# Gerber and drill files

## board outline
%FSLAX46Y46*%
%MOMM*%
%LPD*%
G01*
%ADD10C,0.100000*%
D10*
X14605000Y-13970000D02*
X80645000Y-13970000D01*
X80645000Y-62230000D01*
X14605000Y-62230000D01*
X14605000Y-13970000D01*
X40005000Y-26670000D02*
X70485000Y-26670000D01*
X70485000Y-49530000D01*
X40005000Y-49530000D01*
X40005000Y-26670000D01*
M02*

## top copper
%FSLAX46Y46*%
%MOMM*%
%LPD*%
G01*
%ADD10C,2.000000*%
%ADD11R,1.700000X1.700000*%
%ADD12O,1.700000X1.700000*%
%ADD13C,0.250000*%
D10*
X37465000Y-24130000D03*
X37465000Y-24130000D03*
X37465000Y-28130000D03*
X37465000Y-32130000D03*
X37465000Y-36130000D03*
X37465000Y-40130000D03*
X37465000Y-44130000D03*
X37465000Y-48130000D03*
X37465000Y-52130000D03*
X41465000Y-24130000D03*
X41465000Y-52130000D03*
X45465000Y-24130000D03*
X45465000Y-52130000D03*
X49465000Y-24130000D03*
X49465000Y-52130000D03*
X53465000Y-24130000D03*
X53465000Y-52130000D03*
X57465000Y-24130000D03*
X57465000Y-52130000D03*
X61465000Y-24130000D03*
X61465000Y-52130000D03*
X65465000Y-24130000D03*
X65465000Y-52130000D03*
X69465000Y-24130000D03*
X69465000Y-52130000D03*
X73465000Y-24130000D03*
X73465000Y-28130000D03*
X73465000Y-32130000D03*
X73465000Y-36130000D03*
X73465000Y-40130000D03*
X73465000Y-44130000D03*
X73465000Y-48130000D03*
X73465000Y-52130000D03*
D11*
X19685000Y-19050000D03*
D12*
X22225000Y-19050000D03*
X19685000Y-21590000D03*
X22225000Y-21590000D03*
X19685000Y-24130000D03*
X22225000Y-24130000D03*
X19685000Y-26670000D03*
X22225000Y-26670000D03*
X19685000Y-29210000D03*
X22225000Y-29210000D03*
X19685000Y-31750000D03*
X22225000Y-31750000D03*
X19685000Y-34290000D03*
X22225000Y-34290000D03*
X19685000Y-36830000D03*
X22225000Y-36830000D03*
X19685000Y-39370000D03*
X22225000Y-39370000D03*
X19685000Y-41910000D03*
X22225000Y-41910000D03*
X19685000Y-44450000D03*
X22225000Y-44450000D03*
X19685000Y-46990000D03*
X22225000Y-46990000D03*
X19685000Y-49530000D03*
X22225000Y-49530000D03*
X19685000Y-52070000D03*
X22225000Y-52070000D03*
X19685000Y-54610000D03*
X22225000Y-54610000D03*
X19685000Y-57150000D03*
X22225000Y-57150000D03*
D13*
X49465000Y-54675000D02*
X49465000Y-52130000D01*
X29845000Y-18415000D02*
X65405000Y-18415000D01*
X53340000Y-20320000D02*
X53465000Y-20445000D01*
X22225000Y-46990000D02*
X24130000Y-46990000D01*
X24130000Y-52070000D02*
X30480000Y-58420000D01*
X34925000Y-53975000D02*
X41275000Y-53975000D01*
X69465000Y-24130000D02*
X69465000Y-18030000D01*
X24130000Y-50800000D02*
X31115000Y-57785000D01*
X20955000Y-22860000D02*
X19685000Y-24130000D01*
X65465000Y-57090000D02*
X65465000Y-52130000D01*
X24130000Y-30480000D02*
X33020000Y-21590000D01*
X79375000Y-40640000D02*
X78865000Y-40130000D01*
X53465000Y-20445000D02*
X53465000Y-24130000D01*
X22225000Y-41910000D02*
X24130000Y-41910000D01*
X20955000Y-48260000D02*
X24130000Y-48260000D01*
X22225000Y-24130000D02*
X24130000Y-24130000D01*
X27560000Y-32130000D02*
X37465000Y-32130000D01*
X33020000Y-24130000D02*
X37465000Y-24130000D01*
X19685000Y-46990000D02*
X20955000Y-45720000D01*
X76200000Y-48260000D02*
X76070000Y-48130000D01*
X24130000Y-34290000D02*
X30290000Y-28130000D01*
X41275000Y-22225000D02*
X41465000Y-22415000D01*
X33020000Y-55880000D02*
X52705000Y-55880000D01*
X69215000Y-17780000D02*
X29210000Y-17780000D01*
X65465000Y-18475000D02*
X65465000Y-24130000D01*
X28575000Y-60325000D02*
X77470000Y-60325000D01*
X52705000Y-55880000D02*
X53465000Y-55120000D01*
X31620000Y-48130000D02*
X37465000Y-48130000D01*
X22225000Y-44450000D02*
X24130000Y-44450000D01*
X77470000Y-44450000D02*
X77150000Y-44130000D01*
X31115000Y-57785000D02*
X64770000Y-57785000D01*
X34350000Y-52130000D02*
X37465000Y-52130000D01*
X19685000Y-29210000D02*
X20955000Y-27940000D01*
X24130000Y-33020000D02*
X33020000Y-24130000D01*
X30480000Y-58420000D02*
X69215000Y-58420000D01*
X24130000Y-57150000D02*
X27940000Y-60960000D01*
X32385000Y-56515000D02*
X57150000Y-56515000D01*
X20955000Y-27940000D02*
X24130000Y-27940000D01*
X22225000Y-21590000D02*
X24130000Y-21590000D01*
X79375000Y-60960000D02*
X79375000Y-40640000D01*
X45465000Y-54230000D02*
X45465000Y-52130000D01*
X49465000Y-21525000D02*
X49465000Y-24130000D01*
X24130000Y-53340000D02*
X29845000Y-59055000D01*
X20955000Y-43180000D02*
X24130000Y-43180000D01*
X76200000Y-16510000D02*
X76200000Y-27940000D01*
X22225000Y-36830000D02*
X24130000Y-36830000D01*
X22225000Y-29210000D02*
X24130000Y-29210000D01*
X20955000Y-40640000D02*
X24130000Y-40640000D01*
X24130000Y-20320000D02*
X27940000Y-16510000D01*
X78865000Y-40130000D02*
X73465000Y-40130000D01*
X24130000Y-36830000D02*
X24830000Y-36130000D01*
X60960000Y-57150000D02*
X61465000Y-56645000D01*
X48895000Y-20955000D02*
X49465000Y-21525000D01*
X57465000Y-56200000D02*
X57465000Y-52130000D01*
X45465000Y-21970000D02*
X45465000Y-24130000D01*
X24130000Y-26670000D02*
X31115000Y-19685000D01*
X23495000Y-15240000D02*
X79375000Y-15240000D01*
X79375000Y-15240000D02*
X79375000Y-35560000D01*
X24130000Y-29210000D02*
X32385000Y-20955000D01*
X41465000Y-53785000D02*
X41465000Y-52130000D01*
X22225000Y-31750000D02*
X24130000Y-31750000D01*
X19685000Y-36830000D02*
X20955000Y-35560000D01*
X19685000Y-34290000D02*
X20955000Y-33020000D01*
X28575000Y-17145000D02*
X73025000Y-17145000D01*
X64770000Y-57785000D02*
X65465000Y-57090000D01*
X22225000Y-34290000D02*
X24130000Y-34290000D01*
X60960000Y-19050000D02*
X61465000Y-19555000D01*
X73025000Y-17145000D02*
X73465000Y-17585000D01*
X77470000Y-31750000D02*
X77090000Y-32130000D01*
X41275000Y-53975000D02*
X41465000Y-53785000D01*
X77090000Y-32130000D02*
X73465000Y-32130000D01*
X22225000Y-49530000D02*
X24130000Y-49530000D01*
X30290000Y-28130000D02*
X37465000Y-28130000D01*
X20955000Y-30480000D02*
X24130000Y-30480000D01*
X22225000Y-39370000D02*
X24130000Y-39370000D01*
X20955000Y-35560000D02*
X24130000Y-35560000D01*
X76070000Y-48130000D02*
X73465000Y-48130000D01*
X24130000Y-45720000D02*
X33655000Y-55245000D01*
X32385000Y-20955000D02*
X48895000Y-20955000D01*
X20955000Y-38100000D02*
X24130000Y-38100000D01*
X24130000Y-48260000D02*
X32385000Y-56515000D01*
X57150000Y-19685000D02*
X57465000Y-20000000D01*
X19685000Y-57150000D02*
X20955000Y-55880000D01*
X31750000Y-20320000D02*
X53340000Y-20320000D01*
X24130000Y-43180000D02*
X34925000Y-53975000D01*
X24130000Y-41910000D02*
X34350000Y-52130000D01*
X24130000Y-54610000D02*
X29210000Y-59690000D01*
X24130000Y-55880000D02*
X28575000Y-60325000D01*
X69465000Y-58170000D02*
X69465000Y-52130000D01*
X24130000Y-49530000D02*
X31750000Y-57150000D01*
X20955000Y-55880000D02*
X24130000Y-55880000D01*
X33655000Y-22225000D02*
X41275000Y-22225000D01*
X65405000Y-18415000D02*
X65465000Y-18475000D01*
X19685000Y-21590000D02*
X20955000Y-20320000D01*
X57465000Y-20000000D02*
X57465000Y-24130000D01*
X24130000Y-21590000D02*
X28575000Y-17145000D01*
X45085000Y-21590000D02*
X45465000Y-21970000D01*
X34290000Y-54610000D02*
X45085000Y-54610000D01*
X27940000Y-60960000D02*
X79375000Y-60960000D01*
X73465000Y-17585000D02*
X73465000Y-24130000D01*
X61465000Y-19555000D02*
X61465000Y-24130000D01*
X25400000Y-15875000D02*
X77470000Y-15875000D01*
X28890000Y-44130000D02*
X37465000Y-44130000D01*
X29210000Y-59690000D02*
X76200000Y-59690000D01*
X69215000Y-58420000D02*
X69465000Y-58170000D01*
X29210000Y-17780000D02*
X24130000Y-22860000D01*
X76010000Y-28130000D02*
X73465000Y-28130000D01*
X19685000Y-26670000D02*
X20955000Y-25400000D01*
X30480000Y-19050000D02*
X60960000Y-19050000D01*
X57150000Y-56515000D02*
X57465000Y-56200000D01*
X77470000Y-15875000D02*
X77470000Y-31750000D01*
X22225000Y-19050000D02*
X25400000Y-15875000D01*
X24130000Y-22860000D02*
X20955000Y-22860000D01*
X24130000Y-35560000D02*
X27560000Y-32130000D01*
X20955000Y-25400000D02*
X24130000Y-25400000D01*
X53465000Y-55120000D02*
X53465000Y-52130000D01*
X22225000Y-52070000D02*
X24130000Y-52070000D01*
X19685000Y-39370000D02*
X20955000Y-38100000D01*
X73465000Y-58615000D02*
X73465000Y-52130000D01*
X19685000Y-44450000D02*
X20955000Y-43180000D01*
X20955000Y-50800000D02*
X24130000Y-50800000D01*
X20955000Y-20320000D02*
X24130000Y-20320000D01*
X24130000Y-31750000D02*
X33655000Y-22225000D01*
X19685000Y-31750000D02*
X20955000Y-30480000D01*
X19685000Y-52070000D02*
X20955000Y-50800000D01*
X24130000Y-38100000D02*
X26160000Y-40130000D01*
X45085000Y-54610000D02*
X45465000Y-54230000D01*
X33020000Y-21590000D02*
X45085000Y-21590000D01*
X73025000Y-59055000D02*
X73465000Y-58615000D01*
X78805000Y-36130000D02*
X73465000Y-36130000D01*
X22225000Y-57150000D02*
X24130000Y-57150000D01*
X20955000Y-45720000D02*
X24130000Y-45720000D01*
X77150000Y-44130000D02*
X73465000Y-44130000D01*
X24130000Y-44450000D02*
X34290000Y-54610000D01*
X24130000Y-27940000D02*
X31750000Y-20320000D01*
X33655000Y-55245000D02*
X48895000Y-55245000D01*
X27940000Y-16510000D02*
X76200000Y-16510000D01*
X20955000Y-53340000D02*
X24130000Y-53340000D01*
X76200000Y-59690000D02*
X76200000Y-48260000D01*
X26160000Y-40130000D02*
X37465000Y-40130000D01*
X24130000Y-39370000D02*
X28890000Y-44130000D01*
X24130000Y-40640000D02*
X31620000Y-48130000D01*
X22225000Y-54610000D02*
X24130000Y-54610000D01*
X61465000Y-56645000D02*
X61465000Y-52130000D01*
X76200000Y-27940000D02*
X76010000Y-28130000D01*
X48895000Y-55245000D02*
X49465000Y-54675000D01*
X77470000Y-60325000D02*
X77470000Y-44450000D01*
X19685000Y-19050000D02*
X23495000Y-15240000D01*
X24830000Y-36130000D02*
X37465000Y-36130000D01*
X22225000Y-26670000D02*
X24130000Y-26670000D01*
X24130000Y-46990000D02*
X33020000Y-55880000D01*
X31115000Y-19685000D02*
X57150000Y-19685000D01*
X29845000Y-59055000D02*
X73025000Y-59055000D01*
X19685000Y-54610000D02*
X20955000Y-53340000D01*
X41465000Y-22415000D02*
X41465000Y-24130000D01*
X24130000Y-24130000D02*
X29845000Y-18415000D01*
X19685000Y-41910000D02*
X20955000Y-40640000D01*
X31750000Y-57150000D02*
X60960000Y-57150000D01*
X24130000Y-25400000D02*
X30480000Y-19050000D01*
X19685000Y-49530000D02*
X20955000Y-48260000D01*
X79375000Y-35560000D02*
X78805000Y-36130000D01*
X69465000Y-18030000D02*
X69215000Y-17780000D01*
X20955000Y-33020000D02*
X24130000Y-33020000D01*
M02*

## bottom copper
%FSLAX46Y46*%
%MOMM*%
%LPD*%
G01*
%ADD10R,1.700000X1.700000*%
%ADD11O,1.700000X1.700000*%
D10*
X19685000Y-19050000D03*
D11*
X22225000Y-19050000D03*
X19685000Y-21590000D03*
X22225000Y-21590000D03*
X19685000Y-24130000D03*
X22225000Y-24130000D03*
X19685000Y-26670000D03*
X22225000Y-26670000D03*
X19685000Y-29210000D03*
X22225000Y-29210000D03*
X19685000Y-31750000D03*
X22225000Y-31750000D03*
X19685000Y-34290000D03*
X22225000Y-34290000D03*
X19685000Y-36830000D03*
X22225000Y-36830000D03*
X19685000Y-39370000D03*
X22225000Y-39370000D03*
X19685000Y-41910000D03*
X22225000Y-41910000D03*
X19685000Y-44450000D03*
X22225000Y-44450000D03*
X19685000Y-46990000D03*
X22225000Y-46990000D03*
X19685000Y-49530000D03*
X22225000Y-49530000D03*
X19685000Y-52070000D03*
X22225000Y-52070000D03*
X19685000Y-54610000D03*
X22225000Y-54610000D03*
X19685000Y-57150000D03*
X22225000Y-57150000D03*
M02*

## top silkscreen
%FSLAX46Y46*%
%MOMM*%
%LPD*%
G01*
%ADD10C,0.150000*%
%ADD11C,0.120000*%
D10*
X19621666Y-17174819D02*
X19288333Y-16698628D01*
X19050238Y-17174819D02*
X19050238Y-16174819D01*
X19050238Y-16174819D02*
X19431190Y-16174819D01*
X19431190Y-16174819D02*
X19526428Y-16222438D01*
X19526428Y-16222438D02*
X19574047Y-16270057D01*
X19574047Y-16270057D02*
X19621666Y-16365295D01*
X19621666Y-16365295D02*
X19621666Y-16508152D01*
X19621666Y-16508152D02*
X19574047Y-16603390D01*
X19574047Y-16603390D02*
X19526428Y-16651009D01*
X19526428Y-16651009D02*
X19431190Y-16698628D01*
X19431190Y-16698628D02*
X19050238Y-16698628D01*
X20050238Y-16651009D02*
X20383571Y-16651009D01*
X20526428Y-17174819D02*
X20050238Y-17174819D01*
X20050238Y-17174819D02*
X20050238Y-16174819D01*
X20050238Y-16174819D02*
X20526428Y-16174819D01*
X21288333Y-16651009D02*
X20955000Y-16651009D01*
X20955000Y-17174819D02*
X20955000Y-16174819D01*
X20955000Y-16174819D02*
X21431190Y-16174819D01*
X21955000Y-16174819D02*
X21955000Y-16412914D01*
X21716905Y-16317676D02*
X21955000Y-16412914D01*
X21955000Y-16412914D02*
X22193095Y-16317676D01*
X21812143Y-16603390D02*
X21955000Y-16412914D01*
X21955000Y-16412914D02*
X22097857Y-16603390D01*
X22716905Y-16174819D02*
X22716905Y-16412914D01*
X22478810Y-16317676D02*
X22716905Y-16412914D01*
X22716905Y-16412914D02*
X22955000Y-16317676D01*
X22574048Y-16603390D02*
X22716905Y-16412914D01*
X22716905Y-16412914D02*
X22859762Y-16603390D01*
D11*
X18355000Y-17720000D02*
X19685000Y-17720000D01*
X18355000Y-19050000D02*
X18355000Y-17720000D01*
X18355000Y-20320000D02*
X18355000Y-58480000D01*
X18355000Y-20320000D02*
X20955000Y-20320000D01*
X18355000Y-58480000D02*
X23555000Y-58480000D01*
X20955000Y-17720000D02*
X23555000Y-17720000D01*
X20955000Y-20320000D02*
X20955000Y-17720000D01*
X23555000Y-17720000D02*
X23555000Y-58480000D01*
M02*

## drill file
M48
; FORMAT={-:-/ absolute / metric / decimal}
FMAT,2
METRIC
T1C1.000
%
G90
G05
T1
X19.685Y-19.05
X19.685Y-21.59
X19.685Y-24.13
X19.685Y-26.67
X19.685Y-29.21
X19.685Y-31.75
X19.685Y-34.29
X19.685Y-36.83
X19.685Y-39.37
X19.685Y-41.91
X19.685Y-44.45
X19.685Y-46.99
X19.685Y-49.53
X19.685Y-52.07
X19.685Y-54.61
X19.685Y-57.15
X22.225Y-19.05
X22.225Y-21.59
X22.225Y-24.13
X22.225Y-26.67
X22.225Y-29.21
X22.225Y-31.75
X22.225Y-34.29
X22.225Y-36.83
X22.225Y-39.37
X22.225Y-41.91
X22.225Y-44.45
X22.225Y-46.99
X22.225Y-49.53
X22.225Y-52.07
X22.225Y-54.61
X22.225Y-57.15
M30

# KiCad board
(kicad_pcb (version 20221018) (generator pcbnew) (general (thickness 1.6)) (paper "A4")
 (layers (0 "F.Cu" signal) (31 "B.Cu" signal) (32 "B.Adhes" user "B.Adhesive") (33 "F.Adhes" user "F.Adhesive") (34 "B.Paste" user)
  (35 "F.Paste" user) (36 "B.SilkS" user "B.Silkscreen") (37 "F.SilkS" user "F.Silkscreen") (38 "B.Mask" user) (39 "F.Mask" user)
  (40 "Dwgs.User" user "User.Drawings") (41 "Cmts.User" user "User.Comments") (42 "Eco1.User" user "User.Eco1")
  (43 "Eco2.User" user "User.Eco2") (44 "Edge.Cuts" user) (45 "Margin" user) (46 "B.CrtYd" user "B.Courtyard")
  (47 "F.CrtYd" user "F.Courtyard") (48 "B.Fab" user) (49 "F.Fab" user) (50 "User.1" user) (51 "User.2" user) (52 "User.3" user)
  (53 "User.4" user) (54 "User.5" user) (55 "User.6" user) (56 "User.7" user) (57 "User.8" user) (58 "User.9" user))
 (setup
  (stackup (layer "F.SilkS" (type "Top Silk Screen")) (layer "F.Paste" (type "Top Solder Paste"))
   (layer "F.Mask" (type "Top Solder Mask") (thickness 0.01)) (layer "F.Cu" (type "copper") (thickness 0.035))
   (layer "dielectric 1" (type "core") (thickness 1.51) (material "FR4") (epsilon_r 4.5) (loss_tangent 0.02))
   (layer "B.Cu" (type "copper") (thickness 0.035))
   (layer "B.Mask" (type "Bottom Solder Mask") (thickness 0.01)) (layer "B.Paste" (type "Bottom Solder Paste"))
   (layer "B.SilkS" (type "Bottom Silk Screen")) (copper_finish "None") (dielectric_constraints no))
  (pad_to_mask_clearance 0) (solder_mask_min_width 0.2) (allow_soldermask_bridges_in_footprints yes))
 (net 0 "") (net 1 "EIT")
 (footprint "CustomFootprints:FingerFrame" (layer "F.Cu") (at 37.465 24.13)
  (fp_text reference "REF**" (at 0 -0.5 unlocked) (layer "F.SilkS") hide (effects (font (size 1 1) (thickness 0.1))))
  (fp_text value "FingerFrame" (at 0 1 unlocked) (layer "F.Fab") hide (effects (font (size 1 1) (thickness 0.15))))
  (pad "1" smd circle (at 0 0) (size 2 2) (layers "F.Cu" "F.Paste" "F.Mask") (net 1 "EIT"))
  (pad "1" smd circle (at 0 0) (size 2 2) (layers "F.Cu" "F.Paste" "F.Mask") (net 1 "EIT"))
  (pad "1" smd circle (at 0 4) (size 2 2) (layers "F.Cu" "F.Paste" "F.Mask") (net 1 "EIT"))
  (pad "1" smd circle (at 0 8) (size 2 2) (layers "F.Cu" "F.Paste" "F.Mask") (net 1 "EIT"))
  (pad "1" smd circle (at 0 12) (size 2 2) (layers "F.Cu" "F.Paste" "F.Mask") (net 1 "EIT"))
  (pad "1" smd circle (at 0 16) (size 2 2) (layers "F.Cu" "F.Paste" "F.Mask") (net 1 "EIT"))
  (pad "1" smd circle (at 0 20) (size 2 2) (layers "F.Cu" "F.Paste" "F.Mask") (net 1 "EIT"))
  (pad "1" smd circle (at 0 24) (size 2 2) (layers "F.Cu" "F.Paste" "F.Mask") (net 1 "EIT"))
  (pad "1" smd circle (at 0 28) (size 2 2) (layers "F.Cu" "F.Paste" "F.Mask") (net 1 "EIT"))
  (pad "1" smd circle (at 4 0) (size 2 2) (layers "F.Cu" "F.Paste" "F.Mask") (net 1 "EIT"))
  (pad "1" smd circle (at 4 28) (size 2 2) (layers "F.Cu" "F.Paste" "F.Mask") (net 1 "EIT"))
  (pad "1" smd circle (at 8 0) (size 2 2) (layers "F.Cu" "F.Paste" "F.Mask") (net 1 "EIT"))
  (pad "1" smd circle (at 8 28) (size 2 2) (layers "F.Cu" "F.Paste" "F.Mask") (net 1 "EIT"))
  (pad "1" smd circle (at 12 0) (size 2 2) (layers "F.Cu" "F.Paste" "F.Mask") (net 1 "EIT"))
  (pad "1" smd circle (at 12 28) (size 2 2) (layers "F.Cu" "F.Paste" "F.Mask") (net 1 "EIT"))
  (pad "1" smd circle (at 16 0) (size 2 2) (layers "F.Cu" "F.Paste" "F.Mask") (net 1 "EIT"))
  (pad "1" smd circle (at 16 28) (size 2 2) (layers "F.Cu" "F.Paste" "F.Mask") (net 1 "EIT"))
  (pad "1" smd circle (at 20 0) (size 2 2) (layers "F.Cu" "F.Paste" "F.Mask") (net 1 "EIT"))
  (pad "1" smd circle (at 20 28) (size 2 2) (layers "F.Cu" "F.Paste" "F.Mask") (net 1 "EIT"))
  (pad "1" smd circle (at 24 0) (size 2 2) (layers "F.Cu" "F.Paste" "F.Mask") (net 1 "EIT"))
  (pad "1" smd circle (at 24 28) (size 2 2) (layers "F.Cu" "F.Paste" "F.Mask") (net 1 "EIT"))
  (pad "1" smd circle (at 28 0) (size 2 2) (layers "F.Cu" "F.Paste" "F.Mask") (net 1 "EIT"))
  (pad "1" smd circle (at 28 28) (size 2 2) (layers "F.Cu" "F.Paste" "F.Mask") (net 1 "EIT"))
  (pad "1" smd circle (at 32 0) (size 2 2) (layers "F.Cu" "F.Paste" "F.Mask") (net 1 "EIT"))
  (pad "1" smd circle (at 32 28) (size 2 2) (layers "F.Cu" "F.Paste" "F.Mask") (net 1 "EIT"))
  (pad "1" smd circle (at 36 0) (size 2 2) (layers "F.Cu" "F.Paste" "F.Mask") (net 1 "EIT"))
  (pad "1" smd circle (at 36 4) (size 2 2) (layers "F.Cu" "F.Paste" "F.Mask") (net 1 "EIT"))
  (pad "1" smd circle (at 36 8) (size 2 2) (layers "F.Cu" "F.Paste" "F.Mask") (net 1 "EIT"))
  (pad "1" smd circle (at 36 12) (size 2 2) (layers "F.Cu" "F.Paste" "F.Mask") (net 1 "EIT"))
  (pad "1" smd circle (at 36 16) (size 2 2) (layers "F.Cu" "F.Paste" "F.Mask") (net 1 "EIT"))
  (pad "1" smd circle (at 36 20) (size 2 2) (layers "F.Cu" "F.Paste" "F.Mask") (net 1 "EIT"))
  (pad "1" smd circle (at 36 24) (size 2 2) (layers "F.Cu" "F.Paste" "F.Mask") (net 1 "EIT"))
  (pad "1" smd circle (at 36 28) (size 2 2) (layers "F.Cu" "F.Paste" "F.Mask") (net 1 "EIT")))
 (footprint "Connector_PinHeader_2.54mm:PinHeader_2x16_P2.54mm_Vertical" (layer "F.Cu") (at 19.685 19.05)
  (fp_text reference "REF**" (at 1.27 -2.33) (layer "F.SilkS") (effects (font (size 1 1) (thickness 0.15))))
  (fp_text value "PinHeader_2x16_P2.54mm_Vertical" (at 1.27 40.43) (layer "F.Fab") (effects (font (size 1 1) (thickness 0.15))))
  (fp_line (start -1.33 -1.33) (end 0 -1.33) (stroke (width 0.12) (type solid)) (layer "F.SilkS"))
  (fp_line (start -1.33 0) (end -1.33 -1.33) (stroke (width 0.12) (type solid)) (layer "F.SilkS"))
  (fp_line (start -1.33 1.27) (end -1.33 39.43) (stroke (width 0.12) (type solid)) (layer "F.SilkS"))
  (fp_line (start -1.33 1.27) (end 1.27 1.27) (stroke (width 0.12) (type solid)) (layer "F.SilkS"))
  (fp_line (start -1.33 39.43) (end 3.87 39.43) (stroke (width 0.12) (type solid)) (layer "F.SilkS"))
  (fp_line (start 1.27 -1.33) (end 3.87 -1.33) (stroke (width 0.12) (type solid)) (layer "F.SilkS"))
  (fp_line (start 1.27 1.27) (end 1.27 -1.33) (stroke (width 0.12) (type solid)) (layer "F.SilkS"))
  (fp_line (start 3.87 -1.33) (end 3.87 39.43) (stroke (width 0.12) (type solid)) (layer "F.SilkS"))
  (pad "1" thru_hole rect (at 0 0) (size 1.7 1.7) (drill 1) (layers "*.Cu" "*.Mask") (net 1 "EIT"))
  (pad "2" thru_hole oval (at 2.54 0) (size 1.7 1.7) (drill 1) (layers "*.Cu" "*.Mask") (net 1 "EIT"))
  (pad "3" thru_hole oval (at 0 2.54) (size 1.7 1.7) (drill 1) (layers "*.Cu" "*.Mask") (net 1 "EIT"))
  (pad "4" thru_hole oval (at 2.54 2.54) (size 1.7 1.7) (drill 1) (layers "*.Cu" "*.Mask") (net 1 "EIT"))
  (pad "5" thru_hole oval (at 0 5.08) (size 1.7 1.7) (drill 1) (layers "*.Cu" "*.Mask") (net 1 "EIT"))
  (pad "6" thru_hole oval (at 2.54 5.08) (size 1.7 1.7) (drill 1) (layers "*.Cu" "*.Mask") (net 1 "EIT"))
  (pad "7" thru_hole oval (at 0 7.62) (size 1.7 1.7) (drill 1) (layers "*.Cu" "*.Mask") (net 1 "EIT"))
  (pad "8" thru_hole oval (at 2.54 7.62) (size 1.7 1.7) (drill 1) (layers "*.Cu" "*.Mask") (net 1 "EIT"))
  (pad "9" thru_hole oval (at 0 10.16) (size 1.7 1.7) (drill 1) (layers "*.Cu" "*.Mask") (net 1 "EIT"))
  (pad "10" thru_hole oval (at 2.54 10.16) (size 1.7 1.7) (drill 1) (layers "*.Cu" "*.Mask") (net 1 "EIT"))
  (pad "11" thru_hole oval (at 0 12.7) (size 1.7 1.7) (drill 1) (layers "*.Cu" "*.Mask") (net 1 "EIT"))
  (pad "12" thru_hole oval (at 2.54 12.7) (size 1.7 1.7) (drill 1) (layers "*.Cu" "*.Mask") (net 1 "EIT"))
  (pad "13" thru_hole oval (at 0 15.24) (size 1.7 1.7) (drill 1) (layers "*.Cu" "*.Mask") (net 1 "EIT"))
  (pad "14" thru_hole oval (at 2.54 15.24) (size 1.7 1.7) (drill 1) (layers "*.Cu" "*.Mask") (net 1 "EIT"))
  (pad "15" thru_hole oval (at 0 17.78) (size 1.7 1.7) (drill 1) (layers "*.Cu" "*.Mask") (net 1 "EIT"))
  (pad "16" thru_hole oval (at 2.54 17.78) (size 1.7 1.7) (drill 1) (layers "*.Cu" "*.Mask") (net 1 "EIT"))
  (pad "17" thru_hole oval (at 0 20.32) (size 1.7 1.7) (drill 1) (layers "*.Cu" "*.Mask") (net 1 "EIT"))
  (pad "18" thru_hole oval (at 2.54 20.32) (size 1.7 1.7) (drill 1) (layers "*.Cu" "*.Mask") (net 1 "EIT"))
  (pad "19" thru_hole oval (at 0 22.86) (size 1.7 1.7) (drill 1) (layers "*.Cu" "*.Mask") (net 1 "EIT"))
  (pad "20" thru_hole oval (at 2.54 22.86) (size 1.7 1.7) (drill 1) (layers "*.Cu" "*.Mask") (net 1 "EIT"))
  (pad "21" thru_hole oval (at 0 25.4) (size 1.7 1.7) (drill 1) (layers "*.Cu" "*.Mask") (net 1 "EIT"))
  (pad "22" thru_hole oval (at 2.54 25.4) (size 1.7 1.7) (drill 1) (layers "*.Cu" "*.Mask") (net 1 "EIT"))
  (pad "23" thru_hole oval (at 0 27.94) (size 1.7 1.7) (drill 1) (layers "*.Cu" "*.Mask") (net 1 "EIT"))
  (pad "24" thru_hole oval (at 2.54 27.94) (size 1.7 1.7) (drill 1) (layers "*.Cu" "*.Mask") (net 1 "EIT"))
  (pad "25" thru_hole oval (at 0 30.48) (size 1.7 1.7) (drill 1) (layers "*.Cu" "*.Mask") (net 1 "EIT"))
  (pad "26" thru_hole oval (at 2.54 30.48) (size 1.7 1.7) (drill 1) (layers "*.Cu" "*.Mask") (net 1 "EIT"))
  (pad "27" thru_hole oval (at 0 33.02) (size 1.7 1.7) (drill 1) (layers "*.Cu" "*.Mask") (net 1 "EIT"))
  (pad "28" thru_hole oval (at 2.54 33.02) (size 1.7 1.7) (drill 1) (layers "*.Cu" "*.Mask") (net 1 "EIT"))
  (pad "29" thru_hole oval (at 0 35.56) (size 1.7 1.7) (drill 1) (layers "*.Cu" "*.Mask") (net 1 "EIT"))
  (pad "30" thru_hole oval (at 2.54 35.56) (size 1.7 1.7) (drill 1) (layers "*.Cu" "*.Mask") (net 1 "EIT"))
  (pad "31" thru_hole oval (at 0 38.1) (size 1.7 1.7) (drill 1) (layers "*.Cu" "*.Mask") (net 1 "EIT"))
  (pad "32" thru_hole oval (at 2.54 38.1) (size 1.7 1.7) (drill 1) (layers "*.Cu" "*.Mask") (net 1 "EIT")))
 (gr_rect (start 14.605 13.97) (end 80.645 62.23) (stroke (width 0.1) (type default)) (fill none) (layer "Edge.Cuts"))
 (gr_rect (start 40.005 26.67) (end 70.485 49.53) (stroke (width 0.1) (type default)) (fill none) (layer "Edge.Cuts"))
 (segment (start 49.465 54.675) (end 49.465 52.13) (width 0.25) (layer "F.Cu") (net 1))
 (segment (start 29.845 18.415) (end 65.405 18.415) (width 0.25) (layer "F.Cu") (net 1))
 (segment (start 53.34 20.32) (end 53.465 20.445) (width 0.25) (layer "F.Cu") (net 1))
 (segment (start 22.225 46.99) (end 24.13 46.99) (width 0.25) (layer "F.Cu") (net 1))
 (segment (start 24.13 52.07) (end 30.48 58.42) (width 0.25) (layer "F.Cu") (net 1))
 (segment (start 34.925 53.975) (end 41.275 53.975) (width 0.25) (layer "F.Cu") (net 1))
 (segment (start 69.465 24.13) (end 69.465 18.03) (width 0.25) (layer "F.Cu") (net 1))
 (segment (start 24.13 50.8) (end 31.115 57.785) (width 0.25) (layer "F.Cu") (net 1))
 (segment (start 20.955 22.86) (end 19.685 24.13) (width 0.25) (layer "F.Cu") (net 1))
 (segment (start 65.465 57.09) (end 65.465 52.13) (width 0.25) (layer "F.Cu") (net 1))
 (segment (start 24.13 30.48) (end 33.02 21.59) (width 0.25) (layer "F.Cu") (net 1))
 (segment (start 79.375 40.64) (end 78.865 40.13) (width 0.25) (layer "F.Cu") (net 1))
 (segment (start 53.465 20.445) (end 53.465 24.13) (width 0.25) (layer "F.Cu") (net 1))
 (segment (start 22.225 41.91) (end 24.13 41.91) (width 0.25) (layer "F.Cu") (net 1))
 (segment (start 20.955 48.26) (end 24.13 48.26) (width 0.25) (layer "F.Cu") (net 1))
 (segment (start 22.225 24.13) (end 24.13 24.13) (width 0.25) (layer "F.Cu") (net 1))
 (segment (start 27.56 32.13) (end 37.465 32.13) (width 0.25) (layer "F.Cu") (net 1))
 (segment (start 33.02 24.13) (end 37.465 24.13) (width 0.25) (layer "F.Cu") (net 1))
 (segment (start 19.685 46.99) (end 20.955 45.72) (width 0.25) (layer "F.Cu") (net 1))
 (segment (start 76.2 48.26) (end 76.07 48.13) (width 0.25) (layer "F.Cu") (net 1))
 (segment (start 24.13 34.29) (end 30.29 28.13) (width 0.25) (layer "F.Cu") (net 1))
 (segment (start 41.275 22.225) (end 41.465 22.415) (width 0.25) (layer "F.Cu") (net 1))
 (segment (start 33.02 55.88) (end 52.705 55.88) (width 0.25) (layer "F.Cu") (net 1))
 (segment (start 69.215 17.78) (end 29.21 17.78) (width 0.25) (layer "F.Cu") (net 1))
 (segment (start 65.465 18.475) (end 65.465 24.13) (width 0.25) (layer "F.Cu") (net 1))
 (segment (start 28.575 60.325) (end 77.47 60.325) (width 0.25) (layer "F.Cu") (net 1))
 (segment (start 52.705 55.88) (end 53.465 55.12) (width 0.25) (layer "F.Cu") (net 1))
 (segment (start 31.62 48.13) (end 37.465 48.13) (width 0.25) (layer "F.Cu") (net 1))
 (segment (start 22.225 44.45) (end 24.13 44.45) (width 0.25) (layer "F.Cu") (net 1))
 (segment (start 77.47 44.45) (end 77.15 44.13) (width 0.25) (layer "F.Cu") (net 1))
 (segment (start 31.115 57.785) (end 64.77 57.785) (width 0.25) (layer "F.Cu") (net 1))
 (segment (start 34.35 52.13) (end 37.465 52.13) (width 0.25) (layer "F.Cu") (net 1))
 (segment (start 19.685 29.21) (end 20.955 27.94) (width 0.25) (layer "F.Cu") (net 1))
 (segment (start 24.13 33.02) (end 33.02 24.13) (width 0.25) (layer "F.Cu") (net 1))
 (segment (start 30.48 58.42) (end 69.215 58.42) (width 0.25) (layer "F.Cu") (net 1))
 (segment (start 24.13 57.15) (end 27.94 60.96) (width 0.25) (layer "F.Cu") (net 1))
 (segment (start 32.385 56.515) (end 57.15 56.515) (width 0.25) (layer "F.Cu") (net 1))
 (segment (start 20.955 27.94) (end 24.13 27.94) (width 0.25) (layer "F.Cu") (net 1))
 (segment (start 22.225 21.59) (end 24.13 21.59) (width 0.25) (layer "F.Cu") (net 1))
 (segment (start 79.375 60.96) (end 79.375 40.64) (width 0.25) (layer "F.Cu") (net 1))
 (segment (start 45.465 54.23) (end 45.465 52.13) (width 0.25) (layer "F.Cu") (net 1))
 (segment (start 49.465 21.525) (end 49.465 24.13) (width 0.25) (layer "F.Cu") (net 1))
 (segment (start 24.13 53.34) (end 29.845 59.055) (width 0.25) (layer "F.Cu") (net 1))
 (segment (start 20.955 43.18) (end 24.13 43.18) (width 0.25) (layer "F.Cu") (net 1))
 (segment (start 76.2 16.51) (end 76.2 27.94) (width 0.25) (layer "F.Cu") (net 1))
 (segment (start 22.225 36.83) (end 24.13 36.83) (width 0.25) (layer "F.Cu") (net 1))
 (segment (start 22.225 29.21) (end 24.13 29.21) (width 0.25) (layer "F.Cu") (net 1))
 (segment (start 20.955 40.64) (end 24.13 40.64) (width 0.25) (layer "F.Cu") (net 1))
 (segment (start 24.13 20.32) (end 27.94 16.51) (width 0.25) (layer "F.Cu") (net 1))
 (segment (start 78.865 40.13) (end 73.465 40.13) (width 0.25) (layer "F.Cu") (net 1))
 (segment (start 24.13 36.83) (end 24.83 36.13) (width 0.25) (layer "F.Cu") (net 1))
 (segment (start 60.96 57.15) (end 61.465 56.645) (width 0.25) (layer "F.Cu") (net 1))
 (segment (start 48.895 20.955) (end 49.465 21.525) (width 0.25) (layer "F.Cu") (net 1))
 (segment (start 57.465 56.2) (end 57.465 52.13) (width 0.25) (layer "F.Cu") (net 1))
 (segment (start 45.465 21.97) (end 45.465 24.13) (width 0.25) (layer "F.Cu") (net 1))
 (segment (start 24.13 26.67) (end 31.115 19.685) (width 0.25) (layer "F.Cu") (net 1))
 (segment (start 23.495 15.24) (end 79.375 15.24) (width 0.25) (layer "F.Cu") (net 1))
 (segment (start 79.375 15.24) (end 79.375 35.56) (width 0.25) (layer "F.Cu") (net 1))
 (segment (start 24.13 29.21) (end 32.385 20.955) (width 0.25) (layer "F.Cu") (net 1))
 (segment (start 41.465 53.785) (end 41.465 52.13) (width 0.25) (layer "F.Cu") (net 1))
 (segment (start 22.225 31.75) (end 24.13 31.75) (width 0.25) (layer "F.Cu") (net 1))
 (segment (start 19.685 36.83) (end 20.955 35.56) (width 0.25) (layer "F.Cu") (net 1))
 (segment (start 19.685 34.29) (end 20.955 33.02) (width 0.25) (layer "F.Cu") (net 1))
 (segment (start 28.575 17.145) (end 73.025 17.145) (width 0.25) (layer "F.Cu") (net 1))
 (segment (start 64.77 57.785) (end 65.465 57.09) (width 0.25) (layer "F.Cu") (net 1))
 (segment (start 22.225 34.29) (end 24.13 34.29) (width 0.25) (layer "F.Cu") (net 1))
 (segment (start 60.96 19.05) (end 61.465 19.555) (width 0.25) (layer "F.Cu") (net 1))
 (segment (start 73.025 17.145) (end 73.465 17.585) (width 0.25) (layer "F.Cu") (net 1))
 (segment (start 77.47 31.75) (end 77.09 32.13) (width 0.25) (layer "F.Cu") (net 1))
 (segment (start 41.275 53.975) (end 41.465 53.785) (width 0.25) (layer "F.Cu") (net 1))
 (segment (start 77.09 32.13) (end 73.465 32.13) (width 0.25) (layer "F.Cu") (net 1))
 (segment (start 22.225 49.53) (end 24.13 49.53) (width 0.25) (layer "F.Cu") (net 1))
 (segment (start 30.29 28.13) (end 37.465 28.13) (width 0.25) (layer "F.Cu") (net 1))
 (segment (start 20.955 30.48) (end 24.13 30.48) (width 0.25) (layer "F.Cu") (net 1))
 (segment (start 22.225 39.37) (end 24.13 39.37) (width 0.25) (layer "F.Cu") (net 1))
 (segment (start 20.955 35.56) (end 24.13 35.56) (width 0.25) (layer "F.Cu") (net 1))
 (segment (start 76.07 48.13) (end 73.465 48.13) (width 0.25) (layer "F.Cu") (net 1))
 (segment (start 24.13 45.72) (end 33.655 55.245) (width 0.25) (layer "F.Cu") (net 1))
 (segment (start 32.385 20.955) (end 48.895 20.955) (width 0.25) (layer "F.Cu") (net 1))
 (segment (start 20.955 38.1) (end 24.13 38.1) (width 0.25) (layer "F.Cu") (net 1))
 (segment (start 24.13 48.26) (end 32.385 56.515) (width 0.25) (layer "F.Cu") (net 1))
 (segment (start 57.15 19.685) (end 57.465 20) (width 0.25) (layer "F.Cu") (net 1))
 (segment (start 19.685 57.15) (end 20.955 55.88) (width 0.25) (layer "F.Cu") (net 1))
 (segment (start 31.75 20.32) (end 53.34 20.32) (width 0.25) (layer "F.Cu") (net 1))
 (segment (start 24.13 43.18) (end 34.925 53.975) (width 0.25) (layer "F.Cu") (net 1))
 (segment (start 24.13 41.91) (end 34.35 52.13) (width 0.25) (layer "F.Cu") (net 1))
 (segment (start 24.13 54.61) (end 29.21 59.69) (width 0.25) (layer "F.Cu") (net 1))
 (segment (start 24.13 55.88) (end 28.575 60.325) (width 0.25) (layer "F.Cu") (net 1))
 (segment (start 69.465 58.17) (end 69.465 52.13) (width 0.25) (layer "F.Cu") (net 1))
 (segment (start 24.13 49.53) (end 31.75 57.15) (width 0.25) (layer "F.Cu") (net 1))
 (segment (start 20.955 55.88) (end 24.13 55.88) (width 0.25) (layer "F.Cu") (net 1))
 (segment (start 33.655 22.225) (end 41.275 22.225) (width 0.25) (layer "F.Cu") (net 1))
 (segment (start 65.405 18.415) (end 65.465 18.475) (width 0.25) (layer "F.Cu") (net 1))
 (segment (start 19.685 21.59) (end 20.955 20.32) (width 0.25) (layer "F.Cu") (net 1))
 (segment (start 57.465 20) (end 57.465 24.13) (width 0.25) (layer "F.Cu") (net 1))
 (segment (start 24.13 21.59) (end 28.575 17.145) (width 0.25) (layer "F.Cu") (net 1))
 (segment (start 45.085 21.59) (end 45.465 21.97) (width 0.25) (layer "F.Cu") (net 1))
 (segment (start 34.29 54.61) (end 45.085 54.61) (width 0.25) (layer "F.Cu") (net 1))
 (segment (start 27.94 60.96) (end 79.375 60.96) (width 0.25) (layer "F.Cu") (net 1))
 (segment (start 73.465 17.585) (end 73.465 24.13) (width 0.25) (layer "F.Cu") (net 1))
 (segment (start 61.465 19.555) (end 61.465 24.13) (width 0.25) (layer "F.Cu") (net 1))
 (segment (start 25.4 15.875) (end 77.47 15.875) (width 0.25) (layer "F.Cu") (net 1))
 (segment (start 28.89 44.13) (end 37.465 44.13) (width 0.25) (layer "F.Cu") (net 1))
 (segment (start 29.21 59.69) (end 76.2 59.69) (width 0.25) (layer "F.Cu") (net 1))
 (segment (start 69.215 58.42) (end 69.465 58.17) (width 0.25) (layer "F.Cu") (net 1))
 (segment (start 29.21 17.78) (end 24.13 22.86) (width 0.25) (layer "F.Cu") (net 1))
 (segment (start 76.01 28.13) (end 73.465 28.13) (width 0.25) (layer "F.Cu") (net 1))
 (segment (start 19.685 26.67) (end 20.955 25.4) (width 0.25) (layer "F.Cu") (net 1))
 (segment (start 30.48 19.05) (end 60.96 19.05) (width 0.25) (layer "F.Cu") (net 1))
 (segment (start 57.15 56.515) (end 57.465 56.2) (width 0.25) (layer "F.Cu") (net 1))
 (segment (start 77.47 15.875) (end 77.47 31.75) (width 0.25) (layer "F.Cu") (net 1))
 (segment (start 22.225 19.05) (end 25.4 15.875) (width 0.25) (layer "F.Cu") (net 1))
 (segment (start 24.13 22.86) (end 20.955 22.86) (width 0.25) (layer "F.Cu") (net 1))
 (segment (start 24.13 35.56) (end 27.56 32.13) (width 0.25) (layer "F.Cu") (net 1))
 (segment (start 20.955 25.4) (end 24.13 25.4) (width 0.25) (layer "F.Cu") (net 1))
 (segment (start 53.465 55.12) (end 53.465 52.13) (width 0.25) (layer "F.Cu") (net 1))
 (segment (start 22.225 52.07) (end 24.13 52.07) (width 0.25) (layer "F.Cu") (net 1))
 (segment (start 19.685 39.37) (end 20.955 38.1) (width 0.25) (layer "F.Cu") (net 1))
 (segment (start 73.465 58.615) (end 73.465 52.13) (width 0.25) (layer "F.Cu") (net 1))
 (segment (start 19.685 44.45) (end 20.955 43.18) (width 0.25) (layer "F.Cu") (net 1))
 (segment (start 20.955 50.8) (end 24.13 50.8) (width 0.25) (layer "F.Cu") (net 1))
 (segment (start 20.955 20.32) (end 24.13 20.32) (width 0.25) (layer "F.Cu") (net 1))
 (segment (start 24.13 31.75) (end 33.655 22.225) (width 0.25) (layer "F.Cu") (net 1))
 (segment (start 19.685 31.75) (end 20.955 30.48) (width 0.25) (layer "F.Cu") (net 1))
 (segment (start 19.685 52.07) (end 20.955 50.8) (width 0.25) (layer "F.Cu") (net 1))
 (segment (start 24.13 38.1) (end 26.16 40.13) (width 0.25) (layer "F.Cu") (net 1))
 (segment (start 45.085 54.61) (end 45.465 54.23) (width 0.25) (layer "F.Cu") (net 1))
 (segment (start 33.02 21.59) (end 45.085 21.59) (width 0.25) (layer "F.Cu") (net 1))
 (segment (start 73.025 59.055) (end 73.465 58.615) (width 0.25) (layer "F.Cu") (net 1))
 (segment (start 78.805 36.13) (end 73.465 36.13) (width 0.25) (layer "F.Cu") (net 1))
 (segment (start 22.225 57.15) (end 24.13 57.15) (width 0.25) (layer "F.Cu") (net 1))
 (segment (start 20.955 45.72) (end 24.13 45.72) (width 0.25) (layer "F.Cu") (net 1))
 (segment (start 77.15 44.13) (end 73.465 44.13) (width 0.25) (layer "F.Cu") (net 1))
 (segment (start 24.13 44.45) (end 34.29 54.61) (width 0.25) (layer "F.Cu") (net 1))
 (segment (start 24.13 27.94) (end 31.75 20.32) (width 0.25) (layer "F.Cu") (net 1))
 (segment (start 33.655 55.245) (end 48.895 55.245) (width 0.25) (layer "F.Cu") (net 1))
 (segment (start 27.94 16.51) (end 76.2 16.51) (width 0.25) (layer "F.Cu") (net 1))
 (segment (start 20.955 53.34) (end 24.13 53.34) (width 0.25) (layer "F.Cu") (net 1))
 (segment (start 76.2 59.69) (end 76.2 48.26) (width 0.25) (layer "F.Cu") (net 1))
 (segment (start 26.16 40.13) (end 37.465 40.13) (width 0.25) (layer "F.Cu") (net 1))
 (segment (start 24.13 39.37) (end 28.89 44.13) (width 0.25) (layer "F.Cu") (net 1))
 (segment (start 24.13 40.64) (end 31.62 48.13) (width 0.25) (layer "F.Cu") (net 1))
 (segment (start 22.225 54.61) (end 24.13 54.61) (width 0.25) (layer "F.Cu") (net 1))
 (segment (start 61.465 56.645) (end 61.465 52.13) (width 0.25) (layer "F.Cu") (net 1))
 (segment (start 76.2 27.94) (end 76.01 28.13) (width 0.25) (layer "F.Cu") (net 1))
 (segment (start 48.895 55.245) (end 49.465 54.675) (width 0.25) (layer "F.Cu") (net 1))
 (segment (start 77.47 60.325) (end 77.47 44.45) (width 0.25) (layer "F.Cu") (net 1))
 (segment (start 19.685 19.05) (end 23.495 15.24) (width 0.25) (layer "F.Cu") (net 1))
 (segment (start 24.83 36.13) (end 37.465 36.13) (width 0.25) (layer "F.Cu") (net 1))
 (segment (start 22.225 26.67) (end 24.13 26.67) (width 0.25) (layer "F.Cu") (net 1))
 (segment (start 24.13 46.99) (end 33.02 55.88) (width 0.25) (layer "F.Cu") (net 1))
 (segment (start 31.115 19.685) (end 57.15 19.685) (width 0.25) (layer "F.Cu") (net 1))
 (segment (start 29.845 59.055) (end 73.025 59.055) (width 0.25) (layer "F.Cu") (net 1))
 (segment (start 19.685 54.61) (end 20.955 53.34) (width 0.25) (layer "F.Cu") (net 1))
 (segment (start 41.465 22.415) (end 41.465 24.13) (width 0.25) (layer "F.Cu") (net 1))
 (segment (start 24.13 24.13) (end 29.845 18.415) (width 0.25) (layer "F.Cu") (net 1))
 (segment (start 19.685 41.91) (end 20.955 40.64) (width 0.25) (layer "F.Cu") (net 1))
 (segment (start 31.75 57.15) (end 60.96 57.15) (width 0.25) (layer "F.Cu") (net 1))
 (segment (start 24.13 25.4) (end 30.48 19.05) (width 0.25) (layer "F.Cu") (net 1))
 (segment (start 19.685 49.53) (end 20.955 48.26) (width 0.25) (layer "F.Cu") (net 1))
 (segment (start 79.375 35.56) (end 78.805 36.13) (width 0.25) (layer "F.Cu") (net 1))
 (segment (start 69.465 18.03) (end 69.215 17.78) (width 0.25) (layer "F.Cu") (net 1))
 (segment (start 20.955 33.02) (end 24.13 33.02) (width 0.25) (layer "F.Cu") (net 1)))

